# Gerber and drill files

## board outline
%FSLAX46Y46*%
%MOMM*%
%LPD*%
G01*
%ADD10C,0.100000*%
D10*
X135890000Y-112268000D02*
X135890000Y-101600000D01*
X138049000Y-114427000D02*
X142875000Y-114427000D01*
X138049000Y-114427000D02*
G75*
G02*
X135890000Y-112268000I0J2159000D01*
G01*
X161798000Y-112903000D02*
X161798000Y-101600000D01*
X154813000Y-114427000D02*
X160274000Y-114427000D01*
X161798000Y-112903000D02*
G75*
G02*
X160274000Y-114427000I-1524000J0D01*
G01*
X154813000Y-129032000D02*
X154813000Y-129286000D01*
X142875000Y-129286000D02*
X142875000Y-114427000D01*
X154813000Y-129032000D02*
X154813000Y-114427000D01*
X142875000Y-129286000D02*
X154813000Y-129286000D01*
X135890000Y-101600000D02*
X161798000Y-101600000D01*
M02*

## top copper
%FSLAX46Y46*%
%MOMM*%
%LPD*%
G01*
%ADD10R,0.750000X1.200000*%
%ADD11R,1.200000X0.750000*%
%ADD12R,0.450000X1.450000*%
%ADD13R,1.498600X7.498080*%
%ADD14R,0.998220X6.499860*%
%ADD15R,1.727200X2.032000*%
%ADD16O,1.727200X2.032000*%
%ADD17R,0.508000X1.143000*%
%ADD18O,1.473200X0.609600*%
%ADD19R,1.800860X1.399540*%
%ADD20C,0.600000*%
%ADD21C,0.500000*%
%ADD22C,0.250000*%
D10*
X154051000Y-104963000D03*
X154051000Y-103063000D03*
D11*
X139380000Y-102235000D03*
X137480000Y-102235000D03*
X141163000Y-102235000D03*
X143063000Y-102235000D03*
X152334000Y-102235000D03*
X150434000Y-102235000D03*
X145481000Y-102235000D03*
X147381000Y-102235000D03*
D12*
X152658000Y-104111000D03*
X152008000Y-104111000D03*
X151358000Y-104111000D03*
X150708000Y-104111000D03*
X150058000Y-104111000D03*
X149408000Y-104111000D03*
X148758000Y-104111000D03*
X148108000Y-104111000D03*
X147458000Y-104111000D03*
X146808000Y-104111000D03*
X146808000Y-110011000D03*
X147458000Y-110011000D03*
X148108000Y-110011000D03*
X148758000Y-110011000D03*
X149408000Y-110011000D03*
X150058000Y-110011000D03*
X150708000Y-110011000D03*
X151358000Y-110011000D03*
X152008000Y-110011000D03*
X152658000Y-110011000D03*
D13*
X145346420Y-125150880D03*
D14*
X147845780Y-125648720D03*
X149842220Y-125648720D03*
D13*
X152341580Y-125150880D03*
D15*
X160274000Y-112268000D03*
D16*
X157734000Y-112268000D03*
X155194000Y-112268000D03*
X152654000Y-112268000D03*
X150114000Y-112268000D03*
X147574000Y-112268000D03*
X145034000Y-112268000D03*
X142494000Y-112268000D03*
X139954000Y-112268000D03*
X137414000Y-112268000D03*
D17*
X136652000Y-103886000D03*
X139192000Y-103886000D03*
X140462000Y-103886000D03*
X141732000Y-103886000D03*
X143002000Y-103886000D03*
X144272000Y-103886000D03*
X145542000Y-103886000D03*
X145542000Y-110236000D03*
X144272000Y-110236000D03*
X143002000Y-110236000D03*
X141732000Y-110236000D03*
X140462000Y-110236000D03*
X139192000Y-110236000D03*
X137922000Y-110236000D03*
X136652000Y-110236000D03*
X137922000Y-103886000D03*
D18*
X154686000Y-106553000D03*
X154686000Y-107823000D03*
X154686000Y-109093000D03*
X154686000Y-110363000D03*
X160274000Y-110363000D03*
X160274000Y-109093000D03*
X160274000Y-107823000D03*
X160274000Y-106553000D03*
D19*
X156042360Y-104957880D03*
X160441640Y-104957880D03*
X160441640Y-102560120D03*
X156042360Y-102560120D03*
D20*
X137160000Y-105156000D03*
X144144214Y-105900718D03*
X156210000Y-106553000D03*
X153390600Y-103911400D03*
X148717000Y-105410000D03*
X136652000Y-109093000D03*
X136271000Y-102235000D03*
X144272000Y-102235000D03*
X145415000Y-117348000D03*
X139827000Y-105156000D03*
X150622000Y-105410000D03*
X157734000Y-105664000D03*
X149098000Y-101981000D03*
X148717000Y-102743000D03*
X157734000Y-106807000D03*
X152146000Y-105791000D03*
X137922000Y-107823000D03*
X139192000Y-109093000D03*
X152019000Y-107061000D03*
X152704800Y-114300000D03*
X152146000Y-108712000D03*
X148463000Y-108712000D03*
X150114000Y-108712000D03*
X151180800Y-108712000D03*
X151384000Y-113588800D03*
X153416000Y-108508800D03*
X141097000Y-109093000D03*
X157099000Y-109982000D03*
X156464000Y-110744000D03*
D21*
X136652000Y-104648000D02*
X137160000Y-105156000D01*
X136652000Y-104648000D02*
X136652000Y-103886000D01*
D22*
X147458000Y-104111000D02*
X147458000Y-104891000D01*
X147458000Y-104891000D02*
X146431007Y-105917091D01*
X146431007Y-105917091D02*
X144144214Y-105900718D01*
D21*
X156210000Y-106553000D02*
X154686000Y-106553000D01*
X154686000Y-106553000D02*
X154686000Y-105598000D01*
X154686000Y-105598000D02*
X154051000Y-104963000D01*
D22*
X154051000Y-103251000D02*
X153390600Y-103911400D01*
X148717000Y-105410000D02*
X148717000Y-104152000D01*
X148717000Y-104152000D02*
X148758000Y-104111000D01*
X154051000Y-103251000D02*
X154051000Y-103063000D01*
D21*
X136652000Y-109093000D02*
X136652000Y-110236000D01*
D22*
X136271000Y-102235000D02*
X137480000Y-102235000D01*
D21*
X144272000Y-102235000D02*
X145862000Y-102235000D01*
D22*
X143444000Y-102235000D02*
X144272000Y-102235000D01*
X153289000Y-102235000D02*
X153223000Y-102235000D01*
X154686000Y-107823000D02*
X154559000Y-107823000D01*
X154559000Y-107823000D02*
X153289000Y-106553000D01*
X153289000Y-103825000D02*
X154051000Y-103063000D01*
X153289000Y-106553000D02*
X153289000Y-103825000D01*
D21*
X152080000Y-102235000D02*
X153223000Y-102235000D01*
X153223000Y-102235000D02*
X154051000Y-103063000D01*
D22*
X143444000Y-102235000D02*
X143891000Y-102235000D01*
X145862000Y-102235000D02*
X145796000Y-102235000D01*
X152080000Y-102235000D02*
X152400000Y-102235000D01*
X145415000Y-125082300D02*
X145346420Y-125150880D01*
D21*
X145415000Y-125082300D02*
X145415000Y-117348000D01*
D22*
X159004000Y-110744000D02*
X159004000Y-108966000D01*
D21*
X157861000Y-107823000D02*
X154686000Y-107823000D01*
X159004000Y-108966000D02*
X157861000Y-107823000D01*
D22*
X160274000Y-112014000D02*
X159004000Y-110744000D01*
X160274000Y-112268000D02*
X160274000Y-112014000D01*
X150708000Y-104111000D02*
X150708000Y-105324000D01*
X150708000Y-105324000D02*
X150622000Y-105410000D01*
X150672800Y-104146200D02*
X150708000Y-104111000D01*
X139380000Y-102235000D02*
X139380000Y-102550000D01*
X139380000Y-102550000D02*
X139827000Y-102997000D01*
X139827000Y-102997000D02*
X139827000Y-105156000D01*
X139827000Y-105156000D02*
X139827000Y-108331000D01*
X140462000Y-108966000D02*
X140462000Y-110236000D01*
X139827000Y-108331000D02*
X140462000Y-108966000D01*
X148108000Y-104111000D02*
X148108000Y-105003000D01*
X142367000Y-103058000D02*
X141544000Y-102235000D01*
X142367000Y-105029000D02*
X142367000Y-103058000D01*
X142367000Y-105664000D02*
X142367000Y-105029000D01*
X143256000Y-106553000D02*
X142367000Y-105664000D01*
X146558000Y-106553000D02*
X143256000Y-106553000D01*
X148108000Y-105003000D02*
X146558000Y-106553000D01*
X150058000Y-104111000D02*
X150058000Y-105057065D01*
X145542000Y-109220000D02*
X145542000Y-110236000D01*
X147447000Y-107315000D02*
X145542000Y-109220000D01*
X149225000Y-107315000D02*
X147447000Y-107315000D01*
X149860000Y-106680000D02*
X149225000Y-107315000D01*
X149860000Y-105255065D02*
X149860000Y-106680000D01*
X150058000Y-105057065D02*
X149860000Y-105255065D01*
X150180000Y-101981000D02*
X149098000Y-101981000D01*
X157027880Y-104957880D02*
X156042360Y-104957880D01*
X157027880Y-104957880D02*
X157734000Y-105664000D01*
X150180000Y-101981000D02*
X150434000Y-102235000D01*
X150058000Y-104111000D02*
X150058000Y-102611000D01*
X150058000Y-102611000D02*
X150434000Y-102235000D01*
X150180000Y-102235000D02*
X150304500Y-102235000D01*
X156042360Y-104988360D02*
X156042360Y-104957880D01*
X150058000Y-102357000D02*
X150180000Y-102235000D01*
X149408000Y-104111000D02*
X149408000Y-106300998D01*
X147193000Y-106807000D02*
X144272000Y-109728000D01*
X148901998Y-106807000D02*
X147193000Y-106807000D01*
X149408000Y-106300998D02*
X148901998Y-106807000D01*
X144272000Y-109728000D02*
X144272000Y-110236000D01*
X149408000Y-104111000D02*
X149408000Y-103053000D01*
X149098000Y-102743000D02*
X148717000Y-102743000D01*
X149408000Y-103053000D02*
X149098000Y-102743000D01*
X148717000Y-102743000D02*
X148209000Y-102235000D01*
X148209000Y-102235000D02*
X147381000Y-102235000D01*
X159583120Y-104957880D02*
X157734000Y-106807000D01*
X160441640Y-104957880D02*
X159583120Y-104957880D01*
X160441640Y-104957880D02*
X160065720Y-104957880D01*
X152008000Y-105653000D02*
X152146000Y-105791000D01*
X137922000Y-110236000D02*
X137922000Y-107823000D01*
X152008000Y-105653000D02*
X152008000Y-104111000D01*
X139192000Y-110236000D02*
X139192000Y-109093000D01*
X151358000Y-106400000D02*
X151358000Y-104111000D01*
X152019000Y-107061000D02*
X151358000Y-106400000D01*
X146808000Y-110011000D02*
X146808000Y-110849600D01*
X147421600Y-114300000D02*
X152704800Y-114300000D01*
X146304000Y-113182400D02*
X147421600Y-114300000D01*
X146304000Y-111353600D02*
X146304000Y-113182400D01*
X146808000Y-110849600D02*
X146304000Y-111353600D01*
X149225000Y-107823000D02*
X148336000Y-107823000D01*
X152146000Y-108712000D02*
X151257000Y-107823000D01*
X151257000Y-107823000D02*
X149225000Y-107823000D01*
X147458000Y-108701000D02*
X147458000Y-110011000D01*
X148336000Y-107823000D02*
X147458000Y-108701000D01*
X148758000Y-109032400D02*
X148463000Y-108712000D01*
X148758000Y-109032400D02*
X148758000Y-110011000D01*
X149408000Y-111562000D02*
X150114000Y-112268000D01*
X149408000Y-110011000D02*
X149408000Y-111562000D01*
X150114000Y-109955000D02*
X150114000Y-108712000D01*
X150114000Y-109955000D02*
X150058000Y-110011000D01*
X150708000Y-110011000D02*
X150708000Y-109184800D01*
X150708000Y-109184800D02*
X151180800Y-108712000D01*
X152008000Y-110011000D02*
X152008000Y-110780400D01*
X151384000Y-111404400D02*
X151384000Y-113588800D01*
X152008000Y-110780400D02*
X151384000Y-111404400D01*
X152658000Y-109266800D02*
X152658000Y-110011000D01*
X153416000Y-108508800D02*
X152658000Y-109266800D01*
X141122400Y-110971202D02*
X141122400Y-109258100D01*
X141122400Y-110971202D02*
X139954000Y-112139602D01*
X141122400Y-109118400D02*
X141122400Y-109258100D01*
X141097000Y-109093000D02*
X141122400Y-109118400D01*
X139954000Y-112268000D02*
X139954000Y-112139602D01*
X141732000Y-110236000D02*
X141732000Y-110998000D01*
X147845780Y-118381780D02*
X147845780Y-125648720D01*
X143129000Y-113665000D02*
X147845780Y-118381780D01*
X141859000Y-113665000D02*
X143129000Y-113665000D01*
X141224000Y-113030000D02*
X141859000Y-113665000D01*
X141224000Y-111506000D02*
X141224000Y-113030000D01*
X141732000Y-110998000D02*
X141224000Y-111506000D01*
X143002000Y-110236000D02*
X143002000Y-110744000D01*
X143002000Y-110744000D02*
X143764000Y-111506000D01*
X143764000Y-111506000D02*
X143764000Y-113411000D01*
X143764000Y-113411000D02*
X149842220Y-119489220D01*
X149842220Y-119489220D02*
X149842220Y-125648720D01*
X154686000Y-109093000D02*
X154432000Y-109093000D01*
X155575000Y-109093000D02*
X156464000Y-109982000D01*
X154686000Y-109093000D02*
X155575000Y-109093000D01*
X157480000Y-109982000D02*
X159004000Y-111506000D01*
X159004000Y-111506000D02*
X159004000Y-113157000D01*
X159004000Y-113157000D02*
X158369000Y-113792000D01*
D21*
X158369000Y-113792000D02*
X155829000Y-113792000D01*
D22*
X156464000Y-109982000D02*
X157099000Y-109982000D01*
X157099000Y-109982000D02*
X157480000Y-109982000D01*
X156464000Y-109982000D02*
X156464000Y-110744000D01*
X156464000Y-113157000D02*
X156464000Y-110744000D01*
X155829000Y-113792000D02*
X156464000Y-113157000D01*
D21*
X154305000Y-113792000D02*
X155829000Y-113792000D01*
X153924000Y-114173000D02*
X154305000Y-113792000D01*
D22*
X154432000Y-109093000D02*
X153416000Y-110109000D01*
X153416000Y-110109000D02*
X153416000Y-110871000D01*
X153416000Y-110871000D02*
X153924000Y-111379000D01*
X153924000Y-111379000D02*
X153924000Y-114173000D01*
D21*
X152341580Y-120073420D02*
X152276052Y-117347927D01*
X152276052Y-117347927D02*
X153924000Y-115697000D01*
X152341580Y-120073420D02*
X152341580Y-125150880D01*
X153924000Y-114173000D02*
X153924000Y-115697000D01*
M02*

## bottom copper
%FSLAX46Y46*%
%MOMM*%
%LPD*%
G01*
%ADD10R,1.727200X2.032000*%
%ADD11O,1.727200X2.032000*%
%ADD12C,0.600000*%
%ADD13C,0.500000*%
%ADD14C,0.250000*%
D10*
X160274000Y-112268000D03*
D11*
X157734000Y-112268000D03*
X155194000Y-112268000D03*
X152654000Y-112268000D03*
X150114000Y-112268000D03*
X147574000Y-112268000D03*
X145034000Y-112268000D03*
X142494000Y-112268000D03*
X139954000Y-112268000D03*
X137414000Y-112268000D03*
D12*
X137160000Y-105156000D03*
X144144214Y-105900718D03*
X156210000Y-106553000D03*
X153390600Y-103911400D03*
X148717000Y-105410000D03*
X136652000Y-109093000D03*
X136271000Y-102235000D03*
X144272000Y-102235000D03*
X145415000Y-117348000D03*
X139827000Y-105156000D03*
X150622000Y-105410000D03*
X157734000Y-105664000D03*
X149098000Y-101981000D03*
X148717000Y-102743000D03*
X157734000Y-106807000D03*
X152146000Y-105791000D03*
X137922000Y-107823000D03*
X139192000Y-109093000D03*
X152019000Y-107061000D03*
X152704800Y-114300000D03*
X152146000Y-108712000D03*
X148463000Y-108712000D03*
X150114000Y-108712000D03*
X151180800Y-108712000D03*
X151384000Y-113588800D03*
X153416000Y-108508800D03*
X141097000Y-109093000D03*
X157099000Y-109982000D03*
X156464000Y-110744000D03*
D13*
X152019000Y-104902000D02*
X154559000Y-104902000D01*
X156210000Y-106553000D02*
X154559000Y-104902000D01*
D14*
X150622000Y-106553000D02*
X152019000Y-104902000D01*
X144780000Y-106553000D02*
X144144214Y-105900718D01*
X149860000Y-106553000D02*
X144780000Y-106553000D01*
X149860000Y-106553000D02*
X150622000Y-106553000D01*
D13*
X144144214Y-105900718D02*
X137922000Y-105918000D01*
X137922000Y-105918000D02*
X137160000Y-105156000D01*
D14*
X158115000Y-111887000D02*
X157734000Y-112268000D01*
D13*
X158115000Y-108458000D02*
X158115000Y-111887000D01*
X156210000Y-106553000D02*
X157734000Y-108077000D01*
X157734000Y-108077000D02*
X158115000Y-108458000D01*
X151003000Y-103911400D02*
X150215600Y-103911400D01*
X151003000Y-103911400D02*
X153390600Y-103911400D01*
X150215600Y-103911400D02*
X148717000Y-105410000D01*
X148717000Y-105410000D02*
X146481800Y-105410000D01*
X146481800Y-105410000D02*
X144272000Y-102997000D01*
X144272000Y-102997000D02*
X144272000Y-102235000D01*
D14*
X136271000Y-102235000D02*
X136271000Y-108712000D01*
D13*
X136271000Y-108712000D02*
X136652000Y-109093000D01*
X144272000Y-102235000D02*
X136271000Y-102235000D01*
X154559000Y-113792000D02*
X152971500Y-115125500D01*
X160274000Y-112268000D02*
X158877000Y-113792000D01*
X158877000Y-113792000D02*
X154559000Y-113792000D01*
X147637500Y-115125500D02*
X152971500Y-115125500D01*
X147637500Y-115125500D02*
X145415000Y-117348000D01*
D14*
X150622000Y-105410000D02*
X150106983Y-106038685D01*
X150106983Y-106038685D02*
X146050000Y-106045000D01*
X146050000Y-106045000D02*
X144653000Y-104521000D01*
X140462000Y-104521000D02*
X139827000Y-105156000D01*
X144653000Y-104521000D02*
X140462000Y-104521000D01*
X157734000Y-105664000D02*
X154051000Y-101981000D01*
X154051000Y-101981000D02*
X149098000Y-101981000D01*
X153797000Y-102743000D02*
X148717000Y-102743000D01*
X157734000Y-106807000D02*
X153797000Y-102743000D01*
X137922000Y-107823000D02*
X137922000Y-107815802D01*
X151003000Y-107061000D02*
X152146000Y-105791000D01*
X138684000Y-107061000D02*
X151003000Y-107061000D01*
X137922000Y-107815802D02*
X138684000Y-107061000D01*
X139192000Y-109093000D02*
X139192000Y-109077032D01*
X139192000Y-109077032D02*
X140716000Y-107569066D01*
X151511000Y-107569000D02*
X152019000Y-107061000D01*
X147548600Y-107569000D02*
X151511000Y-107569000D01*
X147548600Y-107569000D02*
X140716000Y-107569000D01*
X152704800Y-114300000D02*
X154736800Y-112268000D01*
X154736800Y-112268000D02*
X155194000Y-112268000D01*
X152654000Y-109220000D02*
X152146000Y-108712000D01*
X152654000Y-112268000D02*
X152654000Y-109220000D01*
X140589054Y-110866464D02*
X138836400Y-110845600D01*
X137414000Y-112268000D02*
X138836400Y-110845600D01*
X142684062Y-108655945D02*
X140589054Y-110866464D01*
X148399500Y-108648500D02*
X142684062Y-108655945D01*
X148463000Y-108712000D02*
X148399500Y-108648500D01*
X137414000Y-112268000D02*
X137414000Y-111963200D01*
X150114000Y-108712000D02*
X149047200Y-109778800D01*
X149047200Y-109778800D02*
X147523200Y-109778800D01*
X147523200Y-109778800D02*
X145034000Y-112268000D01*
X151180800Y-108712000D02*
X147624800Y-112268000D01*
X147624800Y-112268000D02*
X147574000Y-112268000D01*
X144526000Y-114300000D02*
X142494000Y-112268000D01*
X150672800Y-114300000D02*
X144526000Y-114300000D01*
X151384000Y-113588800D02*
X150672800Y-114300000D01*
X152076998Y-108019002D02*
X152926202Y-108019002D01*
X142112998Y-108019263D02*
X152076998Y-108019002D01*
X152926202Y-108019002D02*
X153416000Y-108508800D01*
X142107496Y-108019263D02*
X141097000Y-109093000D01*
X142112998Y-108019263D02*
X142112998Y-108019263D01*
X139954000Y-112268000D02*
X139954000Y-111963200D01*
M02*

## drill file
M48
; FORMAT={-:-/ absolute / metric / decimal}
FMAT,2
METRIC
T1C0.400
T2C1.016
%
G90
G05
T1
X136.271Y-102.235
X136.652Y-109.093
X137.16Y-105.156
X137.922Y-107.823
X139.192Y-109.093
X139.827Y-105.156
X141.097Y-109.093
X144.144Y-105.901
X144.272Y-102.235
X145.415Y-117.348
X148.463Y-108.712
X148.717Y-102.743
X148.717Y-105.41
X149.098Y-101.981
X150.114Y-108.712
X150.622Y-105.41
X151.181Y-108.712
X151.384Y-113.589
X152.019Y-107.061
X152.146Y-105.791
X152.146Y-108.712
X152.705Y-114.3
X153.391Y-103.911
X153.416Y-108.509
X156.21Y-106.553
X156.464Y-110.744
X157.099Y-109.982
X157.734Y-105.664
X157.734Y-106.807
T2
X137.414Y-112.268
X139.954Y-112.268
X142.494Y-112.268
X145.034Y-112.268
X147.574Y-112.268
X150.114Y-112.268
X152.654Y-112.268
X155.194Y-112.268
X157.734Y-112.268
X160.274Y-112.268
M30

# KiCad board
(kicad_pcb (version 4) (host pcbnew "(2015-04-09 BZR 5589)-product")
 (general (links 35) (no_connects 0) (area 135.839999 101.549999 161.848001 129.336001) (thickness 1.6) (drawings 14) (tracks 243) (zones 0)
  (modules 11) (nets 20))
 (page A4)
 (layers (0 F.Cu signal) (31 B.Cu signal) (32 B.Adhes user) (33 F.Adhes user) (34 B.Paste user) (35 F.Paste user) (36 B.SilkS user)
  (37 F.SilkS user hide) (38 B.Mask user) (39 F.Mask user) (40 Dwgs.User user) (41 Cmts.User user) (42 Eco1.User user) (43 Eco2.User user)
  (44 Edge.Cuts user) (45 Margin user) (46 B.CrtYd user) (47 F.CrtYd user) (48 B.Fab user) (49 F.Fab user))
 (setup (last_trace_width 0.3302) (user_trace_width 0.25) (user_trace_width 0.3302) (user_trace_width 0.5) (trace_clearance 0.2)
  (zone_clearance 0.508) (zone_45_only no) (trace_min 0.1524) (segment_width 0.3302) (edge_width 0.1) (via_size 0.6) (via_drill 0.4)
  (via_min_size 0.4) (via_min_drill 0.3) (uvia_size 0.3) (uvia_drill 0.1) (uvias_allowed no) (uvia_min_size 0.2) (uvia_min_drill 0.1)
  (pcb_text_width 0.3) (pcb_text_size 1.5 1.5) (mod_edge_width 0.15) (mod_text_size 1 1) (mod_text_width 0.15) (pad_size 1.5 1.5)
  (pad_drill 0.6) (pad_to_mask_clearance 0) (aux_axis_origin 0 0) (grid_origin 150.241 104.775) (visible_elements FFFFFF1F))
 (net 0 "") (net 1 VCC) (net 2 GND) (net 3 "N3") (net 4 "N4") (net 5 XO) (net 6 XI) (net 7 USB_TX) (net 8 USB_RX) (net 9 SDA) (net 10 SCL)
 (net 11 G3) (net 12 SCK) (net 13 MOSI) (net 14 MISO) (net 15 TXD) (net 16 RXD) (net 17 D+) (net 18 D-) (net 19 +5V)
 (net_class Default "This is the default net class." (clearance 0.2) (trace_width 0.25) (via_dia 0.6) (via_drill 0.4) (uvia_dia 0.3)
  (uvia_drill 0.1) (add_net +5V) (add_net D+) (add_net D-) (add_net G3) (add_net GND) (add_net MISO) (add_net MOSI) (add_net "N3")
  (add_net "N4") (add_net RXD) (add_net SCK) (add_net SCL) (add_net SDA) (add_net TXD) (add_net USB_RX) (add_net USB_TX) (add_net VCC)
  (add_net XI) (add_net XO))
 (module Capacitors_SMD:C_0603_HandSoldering (layer F.Cu) (at 154.051 104.013 90)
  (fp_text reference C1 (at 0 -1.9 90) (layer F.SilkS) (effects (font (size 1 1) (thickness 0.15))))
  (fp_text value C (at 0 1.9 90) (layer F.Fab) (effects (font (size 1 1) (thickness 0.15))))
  (pad 1 smd rect (at -0.95 0 90) (size 1.2 0.75) (layers F.Cu F.Paste F.Mask) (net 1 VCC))
  (pad 2 smd rect (at 0.95 0 90) (size 1.2 0.75) (layers F.Cu F.Paste F.Mask) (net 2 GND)))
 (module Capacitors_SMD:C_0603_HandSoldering (layer F.Cu) (at 138.43 102.235 180)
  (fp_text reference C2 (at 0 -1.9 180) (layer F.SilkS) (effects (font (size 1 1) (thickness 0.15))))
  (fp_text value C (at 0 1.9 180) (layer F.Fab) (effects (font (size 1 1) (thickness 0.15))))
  (pad 1 smd rect (at -0.95 0 180) (size 1.2 0.75) (layers F.Cu F.Paste F.Mask) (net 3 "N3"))
  (pad 2 smd rect (at 0.95 0 180) (size 1.2 0.75) (layers F.Cu F.Paste F.Mask) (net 2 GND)))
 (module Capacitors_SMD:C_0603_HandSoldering (layer F.Cu) (at 142.113 102.235)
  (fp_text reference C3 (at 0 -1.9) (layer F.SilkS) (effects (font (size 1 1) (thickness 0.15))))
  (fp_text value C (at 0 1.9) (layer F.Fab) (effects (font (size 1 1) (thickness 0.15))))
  (pad 1 smd rect (at -0.95 0) (size 1.2 0.75) (layers F.Cu F.Paste F.Mask) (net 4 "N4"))
  (pad 2 smd rect (at 0.95 0) (size 1.2 0.75) (layers F.Cu F.Paste F.Mask) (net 2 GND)))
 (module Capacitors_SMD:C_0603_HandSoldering (layer F.Cu) (at 151.384 102.235 180)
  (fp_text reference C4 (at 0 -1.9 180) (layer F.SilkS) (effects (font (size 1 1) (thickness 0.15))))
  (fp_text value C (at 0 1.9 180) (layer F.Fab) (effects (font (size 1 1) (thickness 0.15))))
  (pad 1 smd rect (at -0.95 0 180) (size 1.2 0.75) (layers F.Cu F.Paste F.Mask) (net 2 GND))
  (pad 2 smd rect (at 0.95 0 180) (size 1.2 0.75) (layers F.Cu F.Paste F.Mask) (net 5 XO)))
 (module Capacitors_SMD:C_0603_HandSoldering (layer F.Cu) (at 146.431 102.235)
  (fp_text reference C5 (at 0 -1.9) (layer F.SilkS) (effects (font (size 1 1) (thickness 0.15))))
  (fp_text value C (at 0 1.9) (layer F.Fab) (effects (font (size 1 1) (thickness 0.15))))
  (pad 1 smd rect (at -0.95 0) (size 1.2 0.75) (layers F.Cu F.Paste F.Mask) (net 2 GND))
  (pad 2 smd rect (at 0.95 0) (size 1.2 0.75) (layers F.Cu F.Paste F.Mask) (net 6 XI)))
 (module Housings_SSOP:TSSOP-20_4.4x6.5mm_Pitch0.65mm (layer F.Cu) (at 149.733 107.061 270)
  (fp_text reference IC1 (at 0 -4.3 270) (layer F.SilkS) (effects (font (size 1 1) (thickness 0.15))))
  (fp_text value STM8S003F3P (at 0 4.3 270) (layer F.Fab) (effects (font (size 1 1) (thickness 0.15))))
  (pad 1 smd rect (at -2.95 -2.925 270) (size 1.45 0.45) (layers F.Cu F.Paste F.Mask))
  (pad 2 smd rect (at -2.95 -2.275 270) (size 1.45 0.45) (layers F.Cu F.Paste F.Mask) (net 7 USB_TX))
  (pad 3 smd rect (at -2.95 -1.625 270) (size 1.45 0.45) (layers F.Cu F.Paste F.Mask) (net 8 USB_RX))
  (pad 4 smd rect (at -2.95 -0.975 270) (size 1.45 0.45) (layers F.Cu F.Paste F.Mask) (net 3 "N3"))
  (pad 5 smd rect (at -2.95 -0.325 270) (size 1.45 0.45) (layers F.Cu F.Paste F.Mask) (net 5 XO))
  (pad 6 smd rect (at -2.95 0.325 270) (size 1.45 0.45) (layers F.Cu F.Paste F.Mask) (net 6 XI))
  (pad 7 smd rect (at -2.95 0.975 270) (size 1.45 0.45) (layers F.Cu F.Paste F.Mask) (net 2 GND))
  (pad 8 smd rect (at -2.95 1.625 270) (size 1.45 0.45) (layers F.Cu F.Paste F.Mask) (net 4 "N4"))
  (pad 9 smd rect (at -2.95 2.275 270) (size 1.45 0.45) (layers F.Cu F.Paste F.Mask) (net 1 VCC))
  (pad 10 smd rect (at -2.95 2.925 270) (size 1.45 0.45) (layers F.Cu F.Paste F.Mask))
  (pad 11 smd rect (at 2.95 2.925 270) (size 1.45 0.45) (layers F.Cu F.Paste F.Mask) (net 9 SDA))
  (pad 12 smd rect (at 2.95 2.275 270) (size 1.45 0.45) (layers F.Cu F.Paste F.Mask) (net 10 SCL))
  (pad 13 smd rect (at 2.95 1.625 270) (size 1.45 0.45) (layers F.Cu F.Paste F.Mask))
  (pad 14 smd rect (at 2.95 0.975 270) (size 1.45 0.45) (layers F.Cu F.Paste F.Mask) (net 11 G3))
  (pad 15 smd rect (at 2.95 0.325 270) (size 1.45 0.45) (layers F.Cu F.Paste F.Mask) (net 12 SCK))
  (pad 16 smd rect (at 2.95 -0.325 270) (size 1.45 0.45) (layers F.Cu F.Paste F.Mask) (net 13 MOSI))
  (pad 17 smd rect (at 2.95 -0.975 270) (size 1.45 0.45) (layers F.Cu F.Paste F.Mask) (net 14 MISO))
  (pad 18 smd rect (at 2.95 -1.625 270) (size 1.45 0.45) (layers F.Cu F.Paste F.Mask))
  (pad 19 smd rect (at 2.95 -2.275 270) (size 1.45 0.45) (layers F.Cu F.Paste F.Mask) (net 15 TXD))
  (pad 20 smd rect (at 2.95 -2.925 270) (size 1.45 0.45) (layers F.Cu F.Paste F.Mask) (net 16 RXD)))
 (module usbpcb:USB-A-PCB (layer F.Cu) (at 148.844 125.349 270)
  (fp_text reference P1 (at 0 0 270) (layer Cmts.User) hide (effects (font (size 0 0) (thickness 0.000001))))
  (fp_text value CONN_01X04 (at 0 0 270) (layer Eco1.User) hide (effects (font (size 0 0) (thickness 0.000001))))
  (pad 4 smd rect (at -0.19812 3.49758 270) (size 7.49808 1.4986) (layers F.Cu F.Paste F.Mask) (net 2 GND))
  (pad 3 smd rect (at 0.29972 0.99822 270) (size 6.49986 0.99822) (layers F.Cu F.Paste F.Mask) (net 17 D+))
  (pad 2 smd rect (at 0.29972 -0.99822 270) (size 6.49986 0.99822) (layers F.Cu F.Paste F.Mask) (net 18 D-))
  (pad 1 smd rect (at -0.19812 -3.49758 270) (size 7.49808 1.4986) (layers F.Cu F.Paste F.Mask) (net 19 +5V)))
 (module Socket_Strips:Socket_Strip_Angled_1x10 (layer F.Cu) (at 160.274 112.268 180)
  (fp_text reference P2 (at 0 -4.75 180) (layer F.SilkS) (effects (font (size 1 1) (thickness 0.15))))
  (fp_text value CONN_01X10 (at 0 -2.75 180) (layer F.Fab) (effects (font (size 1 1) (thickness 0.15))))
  (pad 1 thru_hole rect (at 0 0 180) (size 1.7272 2.032) (drill 1.016) (layers *.Cu *.Mask F.SilkS) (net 2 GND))
  (pad 2 thru_hole oval (at 2.54 0 180) (size 1.7272 2.032) (drill 1.016) (layers *.Cu *.Mask F.SilkS) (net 1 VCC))
  (pad 3 thru_hole oval (at 5.08 0 180) (size 1.7272 2.032) (drill 1.016) (layers *.Cu *.Mask F.SilkS) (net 9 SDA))
  (pad 4 thru_hole oval (at 7.62 0 180) (size 1.7272 2.032) (drill 1.016) (layers *.Cu *.Mask F.SilkS) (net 10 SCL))
  (pad 5 thru_hole oval (at 10.16 0 180) (size 1.7272 2.032) (drill 1.016) (layers *.Cu *.Mask F.SilkS) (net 12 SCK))
  (pad 6 thru_hole oval (at 12.7 0 180) (size 1.7272 2.032) (drill 1.016) (layers *.Cu *.Mask F.SilkS) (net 14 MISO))
  (pad 7 thru_hole oval (at 15.24 0 180) (size 1.7272 2.032) (drill 1.016) (layers *.Cu *.Mask F.SilkS) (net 13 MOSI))
  (pad 8 thru_hole oval (at 17.78 0 180) (size 1.7272 2.032) (drill 1.016) (layers *.Cu *.Mask F.SilkS) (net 15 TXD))
  (pad 9 thru_hole oval (at 20.32 0 180) (size 1.7272 2.032) (drill 1.016) (layers *.Cu *.Mask F.SilkS) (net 16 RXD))
  (pad 10 thru_hole oval (at 22.86 0 180) (size 1.7272 2.032) (drill 1.016) (layers *.Cu *.Mask F.SilkS) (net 11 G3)))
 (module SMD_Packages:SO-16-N (layer F.Cu) (at 141.097 107.061)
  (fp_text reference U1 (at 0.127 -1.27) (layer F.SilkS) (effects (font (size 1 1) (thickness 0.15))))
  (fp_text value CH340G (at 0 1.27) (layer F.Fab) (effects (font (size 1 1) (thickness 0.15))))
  (pad 16 smd rect (at -4.445 -3.175) (size 0.508 1.143) (layers F.Cu F.Paste F.Mask) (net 1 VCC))
  (pad 14 smd rect (at -1.905 -3.175) (size 0.508 1.143) (layers F.Cu F.Paste F.Mask))
  (pad 13 smd rect (at -0.635 -3.175) (size 0.508 1.143) (layers F.Cu F.Paste F.Mask))
  (pad 12 smd rect (at 0.635 -3.175) (size 0.508 1.143) (layers F.Cu F.Paste F.Mask))
  (pad 11 smd rect (at 1.905 -3.175) (size 0.508 1.143) (layers F.Cu F.Paste F.Mask))
  (pad 10 smd rect (at 3.175 -3.175) (size 0.508 1.143) (layers F.Cu F.Paste F.Mask))
  (pad 9 smd rect (at 4.445 -3.175) (size 0.508 1.143) (layers F.Cu F.Paste F.Mask))
  (pad 8 smd rect (at 4.445 3.175) (size 0.508 1.143) (layers F.Cu F.Paste F.Mask) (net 5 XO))
  (pad 7 smd rect (at 3.175 3.175) (size 0.508 1.143) (layers F.Cu F.Paste F.Mask) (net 6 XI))
  (pad 6 smd rect (at 1.905 3.175) (size 0.508 1.143) (layers F.Cu F.Paste F.Mask) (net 18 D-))
  (pad 5 smd rect (at 0.635 3.175) (size 0.508 1.143) (layers F.Cu F.Paste F.Mask) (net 17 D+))
  (pad 4 smd rect (at -0.635 3.175) (size 0.508 1.143) (layers F.Cu F.Paste F.Mask) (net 3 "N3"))
  (pad 3 smd rect (at -1.905 3.175) (size 0.508 1.143) (layers F.Cu F.Paste F.Mask) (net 8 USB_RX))
  (pad 2 smd rect (at -3.175 3.175) (size 0.508 1.143) (layers F.Cu F.Paste F.Mask) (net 7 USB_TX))
  (pad 1 smd rect (at -4.445 3.175) (size 0.508 1.143) (layers F.Cu F.Paste F.Mask) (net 2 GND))
  (pad 15 smd rect (at -3.175 -3.175) (size 0.508 1.143) (layers F.Cu F.Paste F.Mask)))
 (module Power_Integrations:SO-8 (layer F.Cu) (at 157.48 108.458 270)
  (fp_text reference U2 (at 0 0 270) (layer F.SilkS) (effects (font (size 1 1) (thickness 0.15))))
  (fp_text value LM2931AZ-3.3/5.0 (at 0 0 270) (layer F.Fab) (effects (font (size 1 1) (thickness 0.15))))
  (pad 1 smd oval (at -1.905 2.794 270) (size 0.6096 1.4732) (layers F.Cu F.Paste F.Mask) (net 1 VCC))
  (pad 2 smd oval (at -0.635 2.794 270) (size 0.6096 1.4732) (layers F.Cu F.Paste F.Mask) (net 2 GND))
  (pad 3 smd oval (at 0.635 2.794 270) (size 0.6096 1.4732) (layers F.Cu F.Paste F.Mask) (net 19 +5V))
  (pad 4 smd oval (at 1.905 2.794 270) (size 0.6096 1.4732) (layers F.Cu F.Paste F.Mask))
  (pad 5 smd oval (at 1.905 -2.794 270) (size 0.6096 1.4732) (layers F.Cu F.Paste F.Mask))
  (pad 6 smd oval (at 0.635 -2.794 270) (size 0.6096 1.4732) (layers F.Cu F.Paste F.Mask))
  (pad 7 smd oval (at -0.635 -2.794 270) (size 0.6096 1.4732) (layers F.Cu F.Paste F.Mask))
  (pad 8 smd oval (at -1.905 -2.794 270) (size 0.6096 1.4732) (layers F.Cu F.Paste F.Mask)))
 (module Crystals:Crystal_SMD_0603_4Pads (layer F.Cu) (at 158.242 103.759)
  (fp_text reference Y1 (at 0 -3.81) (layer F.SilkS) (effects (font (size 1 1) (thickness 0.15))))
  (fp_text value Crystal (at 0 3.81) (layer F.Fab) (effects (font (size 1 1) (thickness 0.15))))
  (pad 1 smd rect (at -2.19964 1.19888) (size 1.80086 1.39954) (layers F.Cu F.Paste F.Mask) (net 5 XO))
  (pad 2 smd rect (at 2.19964 1.19888) (size 1.80086 1.39954) (layers F.Cu F.Paste F.Mask) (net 6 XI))
  (pad 3 smd rect (at 2.19964 -1.19888) (size 1.80086 1.39954) (layers F.Cu F.Paste F.Mask))
  (pad 4 smd rect (at -2.19964 -1.19888) (size 1.80086 1.39954) (layers F.Cu F.Paste F.Mask)))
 (gr_line (start 135.89 112.268) (end 135.89 101.6) (angle 90) (layer Edge.Cuts) (width 0.1))
 (gr_line (start 138.049 114.427) (end 142.875 114.427) (angle 90) (layer Edge.Cuts) (width 0.1))
 (gr_arc (start 138.049 112.268) (end 138.049 114.427) (angle 90) (layer Edge.Cuts) (width 0.1))
 (gr_line (start 161.798 112.903) (end 161.798 101.6) (angle 90) (layer Edge.Cuts) (width 0.1))
 (gr_line (start 154.813 114.427) (end 160.274 114.427) (angle 90) (layer Edge.Cuts) (width 0.1))
 (gr_arc (start 160.274 112.903) (end 161.798 112.903) (angle 90) (layer Edge.Cuts) (width 0.1))
 (gr_line (start 154.813 129.032) (end 154.813 129.286) (angle 90) (layer Edge.Cuts) (width 0.1))
 (gr_line (start 142.875 129.286) (end 142.875 114.427) (angle 90) (layer Edge.Cuts) (width 0.1))
 (gr_line (start 154.813 129.032) (end 154.813 114.427) (angle 90) (layer Edge.Cuts) (width 0.1))
 (gr_line (start 142.875 129.286) (end 154.813 129.286) (angle 90) (layer Edge.Cuts) (width 0.1))
 (gr_line (start 135.89 101.6) (end 161.798 101.6) (angle 90) (layer Edge.Cuts) (width 0.1))
 (segment (start 152.019 104.902) (end 154.559 104.902) (width 0.5) (layer B.Cu) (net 1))
 (segment (start 156.21 106.553) (end 154.559 104.902) (width 0.5) (layer B.Cu) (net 1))
 (segment (start 150.622 106.553) (end 152.019 104.902) (width 0.25) (layer B.Cu) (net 1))
 (segment (start 144.78 106.553) (end 144.144214 105.900718) (width 0.25) (layer B.Cu) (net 1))
 (segment (start 149.86 106.553) (end 144.78 106.553) (width 0.25) (layer B.Cu) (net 1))
 (segment (start 149.86 106.553) (end 150.622 106.553) (width 0.25) (layer B.Cu) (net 1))
 (segment (start 144.144214 105.900718) (end 137.922 105.918) (width 0.5) (layer B.Cu) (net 1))
 (segment (start 137.922 105.918) (end 137.16 105.156) (width 0.5) (layer B.Cu) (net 1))
 (segment (start 136.652 104.648) (end 137.16 105.156) (width 0.5) (layer F.Cu) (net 1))
 (via (at 137.16 105.156) (size 0.6) (layers F.Cu B.Cu) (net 1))
 (segment (start 136.652 104.648) (end 136.652 103.886) (width 0.5) (layer F.Cu) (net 1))
 (via (at 144.144214 105.900718) (size 0.6) (layers F.Cu B.Cu) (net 1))
 (segment (start 147.458 104.111) (end 147.458 104.891) (width 0.25) (layer F.Cu) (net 1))
 (segment (start 147.458 104.891) (end 146.431007 105.917091) (width 0.25) (layer F.Cu) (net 1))
 (segment (start 146.431007 105.917091) (end 144.144214 105.900718) (width 0.25) (layer F.Cu) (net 1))
 (segment (start 156.21 106.553) (end 154.686 106.553) (width 0.5) (layer F.Cu) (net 1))
 (via (at 156.21 106.553) (size 0.6) (layers F.Cu B.Cu) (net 1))
 (segment (start 154.686 106.553) (end 154.686 105.598) (width 0.5) (layer F.Cu) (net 1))
 (segment (start 154.686 105.598) (end 154.051 104.963) (width 0.5) (layer F.Cu) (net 1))
 (segment (start 158.115 111.887) (end 157.734 112.268) (width 0.25) (layer B.Cu) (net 1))
 (segment (start 158.115 108.458) (end 158.115 111.887) (width 0.5) (layer B.Cu) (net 1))
 (segment (start 156.21 106.553) (end 157.734 108.077) (width 0.5) (layer B.Cu) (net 1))
 (segment (start 157.734 108.077) (end 158.115 108.458) (width 0.5) (layer B.Cu) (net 1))
 (segment (start 151.003 103.9114) (end 150.2156 103.9114) (width 0.5) (layer B.Cu) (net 2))
 (segment (start 151.003 103.9114) (end 153.3906 103.9114) (width 0.5) (layer B.Cu) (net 2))
 (via (at 153.3906 103.9114) (size 0.6) (layers F.Cu B.Cu) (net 2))
 (segment (start 154.051 103.251) (end 153.3906 103.9114) (width 0.25) (layer F.Cu) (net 2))
 (segment (start 150.2156 103.9114) (end 148.717 105.41) (width 0.5) (layer B.Cu) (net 2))
 (segment (start 148.717 105.41) (end 148.717 104.152) (width 0.25) (layer F.Cu) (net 2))
 (via (at 148.717 105.41) (size 0.6) (layers F.Cu B.Cu) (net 2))
 (segment (start 148.717 104.152) (end 148.758 104.111) (width 0.25) (layer F.Cu) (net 2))
 (segment (start 154.051 103.251) (end 154.051 103.063) (width 0.25) (layer F.Cu) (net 2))
 (segment (start 148.717 105.41) (end 146.4818 105.41) (width 0.5) (layer B.Cu) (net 2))
 (segment (start 146.4818 105.41) (end 144.272 102.997) (width 0.5) (layer B.Cu) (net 2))
 (segment (start 144.272 102.997) (end 144.272 102.235) (width 0.5) (layer B.Cu) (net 2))
 (segment (start 136.271 102.235) (end 136.271 108.712) (width 0.25) (layer B.Cu) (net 2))
 (segment (start 136.652 109.093) (end 136.652 110.236) (width 0.5) (layer F.Cu) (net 2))
 (via (at 136.652 109.093) (size 0.6) (layers F.Cu B.Cu) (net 2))
 (segment (start 136.271 108.712) (end 136.652 109.093) (width 0.5) (layer B.Cu) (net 2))
 (segment (start 144.272 102.235) (end 136.271 102.235) (width 0.5) (layer B.Cu) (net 2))
 (segment (start 136.271 102.235) (end 137.48 102.235) (width 0.25) (layer F.Cu) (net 2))
 (via (at 136.271 102.235) (size 0.6) (layers F.Cu B.Cu) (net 2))
 (segment (start 144.272 102.235) (end 145.862 102.235) (width 0.5) (layer F.Cu) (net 2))
 (segment (start 143.444 102.235) (end 144.272 102.235) (width 0.25) (layer F.Cu) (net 2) (status 10))
 (segment (start 153.289 102.235) (end 153.223 102.235) (width 0.25) (layer F.Cu) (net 2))
 (via (at 144.272 102.235) (size 0.6) (layers F.Cu B.Cu) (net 2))
 (segment (start 154.686 107.823) (end 154.559 107.823) (width 0.25) (layer F.Cu) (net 2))
 (segment (start 154.559 107.823) (end 153.289 106.553) (width 0.25) (layer F.Cu) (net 2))
 (segment (start 153.289 103.825) (end 154.051 103.063) (width 0.25) (layer F.Cu) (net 2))
 (segment (start 153.289 106.553) (end 153.289 103.825) (width 0.25) (layer F.Cu) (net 2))
 (segment (start 154.559 113.792) (end 152.9715 115.1255) (width 0.5) (layer B.Cu) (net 2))
 (segment (start 160.274 112.268) (end 158.877 113.792) (width 0.5) (layer B.Cu) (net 2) (status 400000))
 (segment (start 158.877 113.792) (end 154.559 113.792) (width 0.5) (layer B.Cu) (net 2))
 (segment (start 152.08 102.235) (end 153.223 102.235) (width 0.5) (layer F.Cu) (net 2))
 (segment (start 153.223 102.235) (end 154.051 103.063) (width 0.5) (layer F.Cu) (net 2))
 (segment (start 143.444 102.235) (end 143.891 102.235) (width 0.25) (layer F.Cu) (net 2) (status 30))
 (segment (start 145.862 102.235) (end 145.796 102.235) (width 0.25) (layer F.Cu) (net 2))
 (segment (start 152.08 102.235) (end 152.4 102.235) (width 0.25) (layer F.Cu) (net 2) (status 30))
 (segment (start 145.415 125.0823) (end 145.34642 125.15088) (width 0.25) (layer F.Cu) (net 2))
 (segment (start 147.6375 115.1255) (end 152.9715 115.1255) (width 0.5) (layer B.Cu) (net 2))
 (via (at 145.415 117.348) (size 0.6) (layers F.Cu B.Cu) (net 2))
 (segment (start 147.6375 115.1255) (end 145.415 117.348) (width 0.5) (layer B.Cu) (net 2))
 (segment (start 145.415 125.0823) (end 145.415 117.348) (width 0.5) (layer F.Cu) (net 2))
 (segment (start 159.004 110.744) (end 159.004 108.966) (width 0.25) (layer F.Cu) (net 2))
 (segment (start 157.861 107.823) (end 154.686 107.823) (width 0.5) (layer F.Cu) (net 2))
 (segment (start 159.004 108.966) (end 157.861 107.823) (width 0.5) (layer F.Cu) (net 2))
 (segment (start 160.274 112.014) (end 159.004 110.744) (width 0.25) (layer F.Cu) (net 2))
 (segment (start 160.274 112.268) (end 160.274 112.014) (width 0.25) (layer F.Cu) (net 2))
 (segment (start 150.708 104.111) (end 150.708 105.324) (width 0.25) (layer F.Cu) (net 3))
 (via (at 139.827 105.156) (size 0.6) (layers F.Cu B.Cu) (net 3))
 (via (at 150.622 105.41) (size 0.6) (layers F.Cu B.Cu) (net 3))
 (segment (start 150.622 105.41) (end 150.106983 106.038685) (width 0.25) (layer B.Cu) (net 3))
 (segment (start 150.106983 106.038685) (end 146.05 106.045) (width 0.25) (layer B.Cu) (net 3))
 (segment (start 146.05 106.045) (end 144.653 104.521) (width 0.25) (layer B.Cu) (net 3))
 (segment (start 140.462 104.521) (end 139.827 105.156) (width 0.25) (layer B.Cu) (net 3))
 (segment (start 144.653 104.521) (end 140.462 104.521) (width 0.25) (layer B.Cu) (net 3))
 (segment (start 150.708 105.324) (end 150.622 105.41) (width 0.25) (layer F.Cu) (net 3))
 (segment (start 150.6728 104.1462) (end 150.708 104.111) (width 0.25) (layer F.Cu) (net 3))
 (segment (start 139.38 102.235) (end 139.38 102.55) (width 0.25) (layer F.Cu) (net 3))
 (segment (start 139.38 102.55) (end 139.827 102.997) (width 0.25) (layer F.Cu) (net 3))
 (segment (start 139.827 102.997) (end 139.827 105.156) (width 0.25) (layer F.Cu) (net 3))
 (segment (start 139.827 105.156) (end 139.827 108.331) (width 0.25) (layer F.Cu) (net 3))
 (segment (start 140.462 108.966) (end 140.462 110.236) (width 0.25) (layer F.Cu) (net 3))
 (segment (start 139.827 108.331) (end 140.462 108.966) (width 0.25) (layer F.Cu) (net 3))
 (segment (start 148.108 104.111) (end 148.108 105.003) (width 0.25) (layer F.Cu) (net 4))
 (segment (start 142.367 103.058) (end 141.544 102.235) (width 0.25) (layer F.Cu) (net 4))
 (segment (start 142.367 105.029) (end 142.367 103.058) (width 0.25) (layer F.Cu) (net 4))
 (segment (start 142.367 105.664) (end 142.367 105.029) (width 0.25) (layer F.Cu) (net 4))
 (segment (start 143.256 106.553) (end 142.367 105.664) (width 0.25) (layer F.Cu) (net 4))
 (segment (start 146.558 106.553) (end 143.256 106.553) (width 0.25) (layer F.Cu) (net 4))
 (segment (start 148.108 105.003) (end 146.558 106.553) (width 0.25) (layer F.Cu) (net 4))
 (segment (start 150.058 104.111) (end 150.058 105.057065) (width 0.25) (layer F.Cu) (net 5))
 (segment (start 145.542 109.22) (end 145.542 110.236) (width 0.25) (layer F.Cu) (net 5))
 (segment (start 147.447 107.315) (end 145.542 109.22) (width 0.25) (layer F.Cu) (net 5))
 (segment (start 149.225 107.315) (end 147.447 107.315) (width 0.25) (layer F.Cu) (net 5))
 (segment (start 149.86 106.68) (end 149.225 107.315) (width 0.25) (layer F.Cu) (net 5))
 (segment (start 149.86 105.255065) (end 149.86 106.68) (width 0.25) (layer F.Cu) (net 5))
 (segment (start 150.058 105.057065) (end 149.86 105.255065) (width 0.25) (layer F.Cu) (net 5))
 (segment (start 150.18 101.981) (end 149.098 101.981) (width 0.25) (layer F.Cu) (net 5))
 (segment (start 157.02788 104.95788) (end 156.04236 104.95788) (width 0.25) (layer F.Cu) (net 5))
 (segment (start 157.02788 104.95788) (end 157.734 105.664) (width 0.25) (layer F.Cu) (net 5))
 (via (at 157.734 105.664) (size 0.6) (layers F.Cu B.Cu) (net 5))
 (segment (start 157.734 105.664) (end 154.051 101.981) (width 0.25) (layer B.Cu) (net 5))
 (segment (start 154.051 101.981) (end 149.098 101.981) (width 0.25) (layer B.Cu) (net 5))
 (via (at 149.098 101.981) (size 0.6) (layers F.Cu B.Cu) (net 5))
 (segment (start 150.18 101.981) (end 150.434 102.235) (width 0.25) (layer F.Cu) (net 5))
 (segment (start 150.058 104.111) (end 150.058 102.611) (width 0.25) (layer F.Cu) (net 5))
 (segment (start 150.058 102.611) (end 150.434 102.235) (width 0.25) (layer F.Cu) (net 5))
 (segment (start 150.18 102.235) (end 150.3045 102.235) (width 0.25) (layer F.Cu) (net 5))
 (segment (start 156.04236 104.98836) (end 156.04236 104.95788) (width 0.25) (layer F.Cu) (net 5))
 (segment (start 150.058 102.357) (end 150.18 102.235) (width 0.25) (layer F.Cu) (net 5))
 (segment (start 149.408 104.111) (end 149.408 106.300998) (width 0.25) (layer F.Cu) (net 6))
 (segment (start 147.193 106.807) (end 144.272 109.728) (width 0.25) (layer F.Cu) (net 6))
 (segment (start 148.901998 106.807) (end 147.193 106.807) (width 0.25) (layer F.Cu) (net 6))
 (segment (start 149.408 106.300998) (end 148.901998 106.807) (width 0.25) (layer F.Cu) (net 6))
 (segment (start 144.272 109.728) (end 144.272 110.236) (width 0.25) (layer F.Cu) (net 6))
 (segment (start 149.408 104.111) (end 149.408 103.053) (width 0.25) (layer F.Cu) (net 6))
 (segment (start 149.098 102.743) (end 148.717 102.743) (width 0.25) (layer F.Cu) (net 6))
 (segment (start 149.408 103.053) (end 149.098 102.743) (width 0.25) (layer F.Cu) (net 6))
 (segment (start 148.717 102.743) (end 148.209 102.235) (width 0.25) (layer F.Cu) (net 6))
 (segment (start 148.209 102.235) (end 147.381 102.235) (width 0.25) (layer F.Cu) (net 6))
 (segment (start 159.58312 104.95788) (end 157.734 106.807) (width 0.25) (layer F.Cu) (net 6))
 (via (at 148.717 102.743) (size 0.6) (layers F.Cu B.Cu) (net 6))
 (segment (start 153.797 102.743) (end 148.717 102.743) (width 0.25) (layer B.Cu) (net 6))
 (segment (start 157.734 106.807) (end 153.797 102.743) (width 0.25) (layer B.Cu) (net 6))
 (via (at 157.734 106.807) (size 0.6) (layers F.Cu B.Cu) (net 6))
 (segment (start 160.44164 104.95788) (end 159.58312 104.95788) (width 0.25) (layer F.Cu) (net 6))
 (segment (start 160.44164 104.95788) (end 160.06572 104.95788) (width 0.25) (layer F.Cu) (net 6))
 (segment (start 137.922 107.823) (end 137.922 107.815802) (width 0.25) (layer B.Cu) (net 7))
 (segment (start 152.008 105.653) (end 152.146 105.791) (width 0.25) (layer F.Cu) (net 7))
 (via (at 152.146 105.791) (size 0.6) (layers F.Cu B.Cu) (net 7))
 (via (at 137.922 107.823) (size 0.6) (layers F.Cu B.Cu) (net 7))
 (segment (start 137.922 110.236) (end 137.922 107.823) (width 0.25) (layer F.Cu) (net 7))
 (segment (start 152.008 105.653) (end 152.008 104.111) (width 0.25) (layer F.Cu) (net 7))
 (segment (start 151.003 107.061) (end 152.146 105.791) (width 0.25) (layer B.Cu) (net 7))
 (segment (start 138.684 107.061) (end 151.003 107.061) (width 0.25) (layer B.Cu) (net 7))
 (segment (start 137.922 107.815802) (end 138.684 107.061) (width 0.25) (layer B.Cu) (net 7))
 (segment (start 139.192 109.093) (end 139.192 109.077032) (width 0.25) (layer B.Cu) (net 8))
 (via (at 139.192 109.093) (size 0.6) (layers F.Cu B.Cu) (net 8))
 (segment (start 139.192 110.236) (end 139.192 109.093) (width 0.25) (layer F.Cu) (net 8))
 (segment (start 139.192 109.077032) (end 140.716 107.569066) (width 0.25) (layer B.Cu) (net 8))
 (segment (start 151.511 107.569) (end 152.019 107.061) (width 0.25) (layer B.Cu) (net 8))
 (segment (start 147.5486 107.569) (end 151.511 107.569) (width 0.25) (layer B.Cu) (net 8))
 (segment (start 147.5486 107.569) (end 140.716 107.569) (width 0.25) (layer B.Cu) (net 8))
 (segment (start 151.358 106.4) (end 151.358 104.111) (width 0.25) (layer F.Cu) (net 8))
 (segment (start 152.019 107.061) (end 151.358 106.4) (width 0.25) (layer F.Cu) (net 8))
 (via (at 152.019 107.061) (size 0.6) (layers F.Cu B.Cu) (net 8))
 (segment (start 146.808 110.011) (end 146.808 110.8496) (width 0.25) (layer F.Cu) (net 9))
 (segment (start 152.7048 114.3) (end 154.7368 112.268) (width 0.25) (layer B.Cu) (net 9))
 (via (at 152.7048 114.3) (size 0.6) (layers F.Cu B.Cu) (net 9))
 (segment (start 147.4216 114.3) (end 152.7048 114.3) (width 0.25) (layer F.Cu) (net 9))
 (segment (start 146.304 113.1824) (end 147.4216 114.3) (width 0.25) (layer F.Cu) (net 9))
 (segment (start 146.304 111.3536) (end 146.304 113.1824) (width 0.25) (layer F.Cu) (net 9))
 (segment (start 146.808 110.8496) (end 146.304 111.3536) (width 0.25) (layer F.Cu) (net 9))
 (segment (start 154.7368 112.268) (end 155.194 112.268) (width 0.25) (layer B.Cu) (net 9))
 (segment (start 149.225 107.823) (end 148.336 107.823) (width 0.25) (layer F.Cu) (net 10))
 (segment (start 152.654 109.22) (end 152.146 108.712) (width 0.25) (layer B.Cu) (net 10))
 (via (at 152.146 108.712) (size 0.6) (layers F.Cu B.Cu) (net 10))
 (segment (start 152.146 108.712) (end 151.257 107.823) (width 0.25) (layer F.Cu) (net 10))
 (segment (start 151.257 107.823) (end 149.225 107.823) (width 0.25) (layer F.Cu) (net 10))
 (segment (start 152.654 112.268) (end 152.654 109.22) (width 0.25) (layer B.Cu) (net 10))
 (segment (start 147.458 108.701) (end 147.458 110.011) (width 0.25) (layer F.Cu) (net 10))
 (segment (start 148.336 107.823) (end 147.458 108.701) (width 0.25) (layer F.Cu) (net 10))
 (via (at 148.463 108.712) (size 0.6) (layers F.Cu B.Cu) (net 11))
 (segment (start 148.758 109.0324) (end 148.463 108.712) (width 0.25) (layer F.Cu) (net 11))
 (segment (start 140.589054 110.866464) (end 138.8364 110.8456) (width 0.25) (layer B.Cu) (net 11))
 (segment (start 137.414 112.268) (end 138.8364 110.8456) (width 0.25) (layer B.Cu) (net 11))
 (segment (start 148.758 109.0324) (end 148.758 110.011) (width 0.25) (layer F.Cu) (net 11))
 (segment (start 142.684062 108.655945) (end 140.589054 110.866464) (width 0.25) (layer B.Cu) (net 11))
 (segment (start 148.3995 108.6485) (end 142.684062 108.655945) (width 0.25) (layer B.Cu) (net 11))
 (segment (start 148.463 108.712) (end 148.3995 108.6485) (width 0.25) (layer B.Cu) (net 11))
 (segment (start 137.414 112.268) (end 137.414 111.9632) (width 0.25) (layer B.Cu) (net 11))
 (segment (start 149.408 111.562) (end 150.114 112.268) (width 0.25) (layer F.Cu) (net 12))
 (segment (start 149.408 110.011) (end 149.408 111.562) (width 0.25) (layer F.Cu) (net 12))
 (segment (start 150.114 109.955) (end 150.114 108.712) (width 0.25) (layer F.Cu) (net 13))
 (via (at 150.114 108.712) (size 0.6) (layers F.Cu B.Cu) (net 13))
 (segment (start 150.114 108.712) (end 149.0472 109.7788) (width 0.25) (layer B.Cu) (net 13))
 (segment (start 149.0472 109.7788) (end 147.5232 109.7788) (width 0.25) (layer B.Cu) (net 13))
 (segment (start 147.5232 109.7788) (end 145.034 112.268) (width 0.25) (layer B.Cu) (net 13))
 (segment (start 150.114 109.955) (end 150.058 110.011) (width 0.25) (layer F.Cu) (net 13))
 (segment (start 150.708 110.011) (end 150.708 109.1848) (width 0.25) (layer F.Cu) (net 14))
 (segment (start 151.1808 108.712) (end 147.6248 112.268) (width 0.25) (layer B.Cu) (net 14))
 (via (at 151.1808 108.712) (size 0.6) (layers F.Cu B.Cu) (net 14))
 (segment (start 150.708 109.1848) (end 151.1808 108.712) (width 0.25) (layer F.Cu) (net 14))
 (segment (start 147.6248 112.268) (end 147.574 112.268) (width 0.25) (layer B.Cu) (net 14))
 (segment (start 152.008 110.011) (end 152.008 110.7804) (width 0.25) (layer F.Cu) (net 15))
 (segment (start 144.526 114.3) (end 142.494 112.268) (width 0.25) (layer B.Cu) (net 15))
 (segment (start 150.6728 114.3) (end 144.526 114.3) (width 0.25) (layer B.Cu) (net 15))
 (segment (start 151.384 113.5888) (end 150.6728 114.3) (width 0.25) (layer B.Cu) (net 15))
 (via (at 151.384 113.5888) (size 0.6) (layers F.Cu B.Cu) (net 15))
 (segment (start 151.384 111.4044) (end 151.384 113.5888) (width 0.25) (layer F.Cu) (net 15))
 (segment (start 152.008 110.7804) (end 151.384 111.4044) (width 0.25) (layer F.Cu) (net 15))
 (segment (start 152.076998 108.019002) (end 152.926202 108.019002) (width 0.25) (layer B.Cu) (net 16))
 (segment (start 142.112998 108.019263) (end 152.076998 108.019002) (width 0.25) (layer B.Cu) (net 16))
 (segment (start 152.658 109.2668) (end 152.658 110.011) (width 0.25) (layer F.Cu) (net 16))
 (segment (start 153.416 108.5088) (end 152.658 109.2668) (width 0.25) (layer F.Cu) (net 16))
 (via (at 153.416 108.5088) (size 0.6) (layers F.Cu B.Cu) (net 16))
 (segment (start 152.926202 108.019002) (end 153.416 108.5088) (width 0.25) (layer B.Cu) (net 16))
 (segment (start 141.1224 110.971202) (end 141.1224 109.2581) (width 0.25) (layer F.Cu) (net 16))
 (segment (start 141.1224 110.971202) (end 139.954 112.139602) (width 0.25) (layer F.Cu) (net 16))
 (segment (start 141.1224 109.1184) (end 141.1224 109.2581) (width 0.25) (layer F.Cu) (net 16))
 (segment (start 141.097 109.093) (end 141.1224 109.1184) (width 0.25) (layer F.Cu) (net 16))
 (via (at 141.097 109.093) (size 0.6) (layers F.Cu B.Cu) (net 16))
 (segment (start 142.107496 108.019263) (end 141.097 109.093) (width 0.25) (layer B.Cu) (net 16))
 (segment (start 142.112998 108.019263) (end 142.112998 108.019263) (width 0.25) (layer B.Cu) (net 16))
 (segment (start 139.954 112.268) (end 139.954 112.139602) (width 0.25) (layer F.Cu) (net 16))
 (segment (start 139.954 112.268) (end 139.954 111.9632) (width 0.25) (layer B.Cu) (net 16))
 (segment (start 141.732 110.236) (end 141.732 110.998) (width 0.25) (layer F.Cu) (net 17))
 (segment (start 147.84578 118.38178) (end 147.84578 125.64872) (width 0.25) (layer F.Cu) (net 17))
 (segment (start 143.129 113.665) (end 147.84578 118.38178) (width 0.25) (layer F.Cu) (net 17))
 (segment (start 141.859 113.665) (end 143.129 113.665) (width 0.25) (layer F.Cu) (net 17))
 (segment (start 141.224 113.03) (end 141.859 113.665) (width 0.25) (layer F.Cu) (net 17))
 (segment (start 141.224 111.506) (end 141.224 113.03) (width 0.25) (layer F.Cu) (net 17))
 (segment (start 141.732 110.998) (end 141.224 111.506) (width 0.25) (layer F.Cu) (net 17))
 (segment (start 143.002 110.236) (end 143.002 110.744) (width 0.25) (layer F.Cu) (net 18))
 (segment (start 143.002 110.744) (end 143.764 111.506) (width 0.25) (layer F.Cu) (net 18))
 (segment (start 143.764 111.506) (end 143.764 113.411) (width 0.25) (layer F.Cu) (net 18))
 (segment (start 143.764 113.411) (end 149.84222 119.48922) (width 0.25) (layer F.Cu) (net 18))
 (segment (start 149.84222 119.48922) (end 149.84222 125.64872) (width 0.25) (layer F.Cu) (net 18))
 (segment (start 154.686 109.093) (end 154.432 109.093) (width 0.25) (layer F.Cu) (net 19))
 (segment (start 155.575 109.093) (end 156.464 109.982) (width 0.25) (layer F.Cu) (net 19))
 (segment (start 154.686 109.093) (end 155.575 109.093) (width 0.25) (layer F.Cu) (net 19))
 (segment (start 157.48 109.982) (end 159.004 111.506) (width 0.25) (layer F.Cu) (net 19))
 (segment (start 159.004 111.506) (end 159.004 113.157) (width 0.25) (layer F.Cu) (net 19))
 (segment (start 159.004 113.157) (end 158.369 113.792) (width 0.25) (layer F.Cu) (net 19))
 (segment (start 158.369 113.792) (end 155.829 113.792) (width 0.5) (layer F.Cu) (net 19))
 (segment (start 156.464 109.982) (end 157.099 109.982) (width 0.25) (layer F.Cu) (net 19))
 (via (at 157.099 109.982) (size 0.6) (layers F.Cu B.Cu) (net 19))
 (segment (start 157.099 109.982) (end 157.48 109.982) (width 0.25) (layer F.Cu) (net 19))
 (via (at 156.464 110.744) (size 0.6) (layers F.Cu B.Cu) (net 19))
 (segment (start 156.464 109.982) (end 156.464 110.744) (width 0.25) (layer F.Cu) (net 19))
 (segment (start 156.464 113.157) (end 156.464 110.744) (width 0.25) (layer F.Cu) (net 19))
 (segment (start 155.829 113.792) (end 156.464 113.157) (width 0.25) (layer F.Cu) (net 19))
 (segment (start 154.305 113.792) (end 155.829 113.792) (width 0.5) (layer F.Cu) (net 19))
 (segment (start 153.924 114.173) (end 154.305 113.792) (width 0.5) (layer F.Cu) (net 19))
 (segment (start 154.432 109.093) (end 153.416 110.109) (width 0.25) (layer F.Cu) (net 19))
 (segment (start 153.416 110.109) (end 153.416 110.871) (width 0.25) (layer F.Cu) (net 19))
 (segment (start 153.416 110.871) (end 153.924 111.379) (width 0.25) (layer F.Cu) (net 19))
 (segment (start 153.924 111.379) (end 153.924 114.173) (width 0.25) (layer F.Cu) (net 19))
 (segment (start 152.34158 120.07342) (end 152.276052 117.347927) (width 0.5) (layer F.Cu) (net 19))
 (segment (start 152.276052 117.347927) (end 153.924 115.697) (width 0.5) (layer F.Cu) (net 19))
 (segment (start 152.34158 120.07342) (end 152.34158 125.15088) (width 0.5) (layer F.Cu) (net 19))
 (segment (start 153.924 114.173) (end 153.924 115.697) (width 0.5) (layer F.Cu) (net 19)))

